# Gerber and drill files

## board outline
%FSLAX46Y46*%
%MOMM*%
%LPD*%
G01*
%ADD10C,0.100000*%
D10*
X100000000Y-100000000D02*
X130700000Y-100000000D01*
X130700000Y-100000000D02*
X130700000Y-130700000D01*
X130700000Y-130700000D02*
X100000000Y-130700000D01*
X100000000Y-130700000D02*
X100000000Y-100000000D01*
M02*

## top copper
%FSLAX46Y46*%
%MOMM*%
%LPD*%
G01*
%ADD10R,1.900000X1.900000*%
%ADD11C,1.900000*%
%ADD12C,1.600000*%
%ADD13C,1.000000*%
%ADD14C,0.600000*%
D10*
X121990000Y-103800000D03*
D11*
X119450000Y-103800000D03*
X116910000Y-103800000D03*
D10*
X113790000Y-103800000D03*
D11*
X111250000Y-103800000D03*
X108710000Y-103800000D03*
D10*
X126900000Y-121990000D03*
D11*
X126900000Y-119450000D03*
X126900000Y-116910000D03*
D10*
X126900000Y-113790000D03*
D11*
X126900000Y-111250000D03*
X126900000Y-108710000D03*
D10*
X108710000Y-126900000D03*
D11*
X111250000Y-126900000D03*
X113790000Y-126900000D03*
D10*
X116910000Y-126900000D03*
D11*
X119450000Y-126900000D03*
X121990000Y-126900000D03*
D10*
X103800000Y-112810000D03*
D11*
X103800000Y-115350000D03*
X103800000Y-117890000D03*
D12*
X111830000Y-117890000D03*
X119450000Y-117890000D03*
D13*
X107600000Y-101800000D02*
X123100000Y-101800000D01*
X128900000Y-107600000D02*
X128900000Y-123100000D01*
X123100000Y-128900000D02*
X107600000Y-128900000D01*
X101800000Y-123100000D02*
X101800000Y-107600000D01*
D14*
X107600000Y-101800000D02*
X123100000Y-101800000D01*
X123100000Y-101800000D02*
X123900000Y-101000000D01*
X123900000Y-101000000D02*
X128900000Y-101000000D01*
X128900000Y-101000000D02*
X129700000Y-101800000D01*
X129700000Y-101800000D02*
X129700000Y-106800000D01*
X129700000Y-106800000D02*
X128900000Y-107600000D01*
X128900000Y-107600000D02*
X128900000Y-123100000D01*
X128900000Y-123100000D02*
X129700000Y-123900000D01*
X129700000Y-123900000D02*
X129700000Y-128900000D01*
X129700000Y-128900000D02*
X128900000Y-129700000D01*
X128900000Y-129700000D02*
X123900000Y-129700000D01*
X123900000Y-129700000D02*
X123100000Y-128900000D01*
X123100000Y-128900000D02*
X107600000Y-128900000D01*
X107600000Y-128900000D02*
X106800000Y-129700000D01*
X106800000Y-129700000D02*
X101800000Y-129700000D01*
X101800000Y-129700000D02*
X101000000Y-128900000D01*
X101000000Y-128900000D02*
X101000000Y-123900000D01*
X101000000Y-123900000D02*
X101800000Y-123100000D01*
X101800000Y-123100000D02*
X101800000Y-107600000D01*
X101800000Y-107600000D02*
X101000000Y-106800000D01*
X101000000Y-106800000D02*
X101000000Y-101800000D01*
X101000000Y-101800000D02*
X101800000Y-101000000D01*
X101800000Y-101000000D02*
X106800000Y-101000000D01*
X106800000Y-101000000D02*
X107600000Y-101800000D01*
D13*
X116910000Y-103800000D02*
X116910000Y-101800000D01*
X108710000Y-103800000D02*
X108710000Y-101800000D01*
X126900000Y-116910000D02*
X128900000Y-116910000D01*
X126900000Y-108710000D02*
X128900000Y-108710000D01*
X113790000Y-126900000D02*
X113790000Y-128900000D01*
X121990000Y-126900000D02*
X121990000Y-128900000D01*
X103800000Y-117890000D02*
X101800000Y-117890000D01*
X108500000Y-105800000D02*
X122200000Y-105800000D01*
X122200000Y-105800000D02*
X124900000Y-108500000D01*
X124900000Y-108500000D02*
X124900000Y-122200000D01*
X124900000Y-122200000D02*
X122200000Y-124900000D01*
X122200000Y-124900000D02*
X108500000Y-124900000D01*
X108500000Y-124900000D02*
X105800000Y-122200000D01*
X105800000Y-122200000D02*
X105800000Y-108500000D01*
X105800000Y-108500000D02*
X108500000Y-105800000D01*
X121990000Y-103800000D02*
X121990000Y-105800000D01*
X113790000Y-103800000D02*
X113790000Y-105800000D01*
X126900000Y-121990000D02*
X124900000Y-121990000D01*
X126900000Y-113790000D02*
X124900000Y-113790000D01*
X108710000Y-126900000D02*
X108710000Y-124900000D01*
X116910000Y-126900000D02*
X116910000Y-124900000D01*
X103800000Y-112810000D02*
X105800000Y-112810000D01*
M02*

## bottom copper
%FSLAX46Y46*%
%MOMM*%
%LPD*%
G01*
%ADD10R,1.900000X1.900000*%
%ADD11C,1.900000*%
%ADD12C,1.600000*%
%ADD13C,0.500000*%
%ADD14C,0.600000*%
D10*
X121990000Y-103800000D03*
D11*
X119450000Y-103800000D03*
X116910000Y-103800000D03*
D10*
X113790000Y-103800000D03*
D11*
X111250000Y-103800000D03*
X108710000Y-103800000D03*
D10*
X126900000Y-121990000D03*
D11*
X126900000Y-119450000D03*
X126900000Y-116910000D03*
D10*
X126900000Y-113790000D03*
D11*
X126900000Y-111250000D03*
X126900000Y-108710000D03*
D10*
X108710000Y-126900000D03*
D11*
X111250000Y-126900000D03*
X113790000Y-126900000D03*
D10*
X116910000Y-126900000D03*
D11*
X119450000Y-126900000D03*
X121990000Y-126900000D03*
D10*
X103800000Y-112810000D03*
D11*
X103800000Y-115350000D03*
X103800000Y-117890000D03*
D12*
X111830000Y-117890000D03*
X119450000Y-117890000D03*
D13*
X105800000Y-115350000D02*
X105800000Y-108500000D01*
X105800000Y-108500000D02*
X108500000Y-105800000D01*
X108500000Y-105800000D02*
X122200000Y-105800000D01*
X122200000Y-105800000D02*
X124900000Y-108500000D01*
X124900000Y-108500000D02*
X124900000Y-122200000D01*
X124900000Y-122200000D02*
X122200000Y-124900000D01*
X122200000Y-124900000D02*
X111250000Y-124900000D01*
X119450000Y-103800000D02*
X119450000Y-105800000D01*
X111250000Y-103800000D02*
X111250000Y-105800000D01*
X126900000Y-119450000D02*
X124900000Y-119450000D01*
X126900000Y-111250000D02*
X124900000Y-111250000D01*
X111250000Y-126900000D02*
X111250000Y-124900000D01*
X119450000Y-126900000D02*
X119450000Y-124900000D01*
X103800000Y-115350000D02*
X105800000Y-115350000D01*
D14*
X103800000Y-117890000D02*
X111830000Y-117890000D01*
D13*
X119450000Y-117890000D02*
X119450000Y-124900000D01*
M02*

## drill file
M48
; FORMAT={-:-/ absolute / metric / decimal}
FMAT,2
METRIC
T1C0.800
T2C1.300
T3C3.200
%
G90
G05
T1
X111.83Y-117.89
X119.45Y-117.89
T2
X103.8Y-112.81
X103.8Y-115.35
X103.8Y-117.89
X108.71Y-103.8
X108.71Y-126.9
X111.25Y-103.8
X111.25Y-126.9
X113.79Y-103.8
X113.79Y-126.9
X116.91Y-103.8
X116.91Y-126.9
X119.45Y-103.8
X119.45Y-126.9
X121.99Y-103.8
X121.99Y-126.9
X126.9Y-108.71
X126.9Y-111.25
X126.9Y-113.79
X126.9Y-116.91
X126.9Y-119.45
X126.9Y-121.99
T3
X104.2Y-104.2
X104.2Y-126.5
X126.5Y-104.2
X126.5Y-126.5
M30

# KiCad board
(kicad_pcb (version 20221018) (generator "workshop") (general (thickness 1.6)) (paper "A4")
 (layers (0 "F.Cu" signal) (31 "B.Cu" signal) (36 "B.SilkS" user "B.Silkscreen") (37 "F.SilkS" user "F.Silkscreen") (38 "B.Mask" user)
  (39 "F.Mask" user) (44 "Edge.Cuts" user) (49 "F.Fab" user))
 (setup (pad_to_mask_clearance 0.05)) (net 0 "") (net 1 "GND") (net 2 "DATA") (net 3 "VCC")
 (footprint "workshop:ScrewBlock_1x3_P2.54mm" (layer "F.Cu") (at 121.990 103.800 180)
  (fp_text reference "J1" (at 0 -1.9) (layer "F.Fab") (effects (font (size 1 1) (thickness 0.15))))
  (pad "1" thru_hole rect (at 0.000 0 180) (size 1.9 1.9) (drill 1.3) (layers "*.Cu" "*.Mask") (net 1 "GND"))
  (pad "2" thru_hole circle (at 2.540 0 180) (size 1.9 1.9) (drill 1.3) (layers "*.Cu" "*.Mask") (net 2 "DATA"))
  (pad "3" thru_hole circle (at 5.080 0 180) (size 1.9 1.9) (drill 1.3) (layers "*.Cu" "*.Mask") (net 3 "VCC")))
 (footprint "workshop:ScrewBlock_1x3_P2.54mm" (layer "F.Cu") (at 113.790 103.800 180)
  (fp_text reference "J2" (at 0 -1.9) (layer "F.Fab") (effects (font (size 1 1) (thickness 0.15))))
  (pad "1" thru_hole rect (at 0.000 0 180) (size 1.9 1.9) (drill 1.3) (layers "*.Cu" "*.Mask") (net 1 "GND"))
  (pad "2" thru_hole circle (at 2.540 0 180) (size 1.9 1.9) (drill 1.3) (layers "*.Cu" "*.Mask") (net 2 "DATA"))
  (pad "3" thru_hole circle (at 5.080 0 180) (size 1.9 1.9) (drill 1.3) (layers "*.Cu" "*.Mask") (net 3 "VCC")))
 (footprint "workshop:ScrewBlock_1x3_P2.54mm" (layer "F.Cu") (at 126.900 121.990 90)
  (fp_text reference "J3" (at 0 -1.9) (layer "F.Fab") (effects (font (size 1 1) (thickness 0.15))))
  (pad "1" thru_hole rect (at 0.000 0 90) (size 1.9 1.9) (drill 1.3) (layers "*.Cu" "*.Mask") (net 1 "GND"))
  (pad "2" thru_hole circle (at 2.540 0 90) (size 1.9 1.9) (drill 1.3) (layers "*.Cu" "*.Mask") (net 2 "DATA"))
  (pad "3" thru_hole circle (at 5.080 0 90) (size 1.9 1.9) (drill 1.3) (layers "*.Cu" "*.Mask") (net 3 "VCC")))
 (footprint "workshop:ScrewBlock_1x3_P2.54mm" (layer "F.Cu") (at 126.900 113.790 90)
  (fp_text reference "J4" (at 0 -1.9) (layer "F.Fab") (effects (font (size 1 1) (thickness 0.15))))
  (pad "1" thru_hole rect (at 0.000 0 90) (size 1.9 1.9) (drill 1.3) (layers "*.Cu" "*.Mask") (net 1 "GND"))
  (pad "2" thru_hole circle (at 2.540 0 90) (size 1.9 1.9) (drill 1.3) (layers "*.Cu" "*.Mask") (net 2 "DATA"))
  (pad "3" thru_hole circle (at 5.080 0 90) (size 1.9 1.9) (drill 1.3) (layers "*.Cu" "*.Mask") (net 3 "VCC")))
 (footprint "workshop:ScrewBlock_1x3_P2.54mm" (layer "F.Cu") (at 108.710 126.900 0)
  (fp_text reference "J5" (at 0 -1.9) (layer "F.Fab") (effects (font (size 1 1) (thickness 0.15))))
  (pad "1" thru_hole rect (at 0.000 0 0) (size 1.9 1.9) (drill 1.3) (layers "*.Cu" "*.Mask") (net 1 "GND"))
  (pad "2" thru_hole circle (at 2.540 0 0) (size 1.9 1.9) (drill 1.3) (layers "*.Cu" "*.Mask") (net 2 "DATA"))
  (pad "3" thru_hole circle (at 5.080 0 0) (size 1.9 1.9) (drill 1.3) (layers "*.Cu" "*.Mask") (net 3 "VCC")))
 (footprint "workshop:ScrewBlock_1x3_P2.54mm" (layer "F.Cu") (at 116.910 126.900 0)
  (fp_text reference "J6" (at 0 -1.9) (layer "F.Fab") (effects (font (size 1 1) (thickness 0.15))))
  (pad "1" thru_hole rect (at 0.000 0 0) (size 1.9 1.9) (drill 1.3) (layers "*.Cu" "*.Mask") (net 1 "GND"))
  (pad "2" thru_hole circle (at 2.540 0 0) (size 1.9 1.9) (drill 1.3) (layers "*.Cu" "*.Mask") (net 2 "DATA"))
  (pad "3" thru_hole circle (at 5.080 0 0) (size 1.9 1.9) (drill 1.3) (layers "*.Cu" "*.Mask") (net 3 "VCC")))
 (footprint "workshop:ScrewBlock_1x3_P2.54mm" (layer "F.Cu") (at 103.800 112.810 270)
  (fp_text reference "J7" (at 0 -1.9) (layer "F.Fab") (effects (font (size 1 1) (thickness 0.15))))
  (pad "1" thru_hole rect (at 0.000 0 270) (size 1.9 1.9) (drill 1.3) (layers "*.Cu" "*.Mask") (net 1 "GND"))
  (pad "2" thru_hole circle (at 2.540 0 270) (size 1.9 1.9) (drill 1.3) (layers "*.Cu" "*.Mask") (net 2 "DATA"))
  (pad "3" thru_hole circle (at 5.080 0 270) (size 1.9 1.9) (drill 1.3) (layers "*.Cu" "*.Mask") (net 3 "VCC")))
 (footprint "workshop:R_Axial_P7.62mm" (layer "F.Cu") (at 111.830 117.890)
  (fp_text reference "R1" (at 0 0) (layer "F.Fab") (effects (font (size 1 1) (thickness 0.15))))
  (pad "1" thru_hole circle (at 0.000 0.000) (size 1.6 1.6) (drill 0.8) (layers "*.Cu" "*.Mask") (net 3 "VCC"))
  (pad "2" thru_hole circle (at 7.620 0.000) (size 1.6 1.6) (drill 0.8) (layers "*.Cu" "*.Mask") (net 2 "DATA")))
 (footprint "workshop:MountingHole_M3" (layer "F.Cu") (at 104.200 104.200)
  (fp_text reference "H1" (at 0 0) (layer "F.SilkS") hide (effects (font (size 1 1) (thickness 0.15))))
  (pad "" np_thru_hole circle (at 0 0) (size 3.2 3.2) (drill 3.2) (layers "*.Cu" "*.Mask")))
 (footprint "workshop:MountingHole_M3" (layer "F.Cu") (at 126.500 104.200)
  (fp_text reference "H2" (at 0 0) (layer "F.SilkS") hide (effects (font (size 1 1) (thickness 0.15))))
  (pad "" np_thru_hole circle (at 0 0) (size 3.2 3.2) (drill 3.2) (layers "*.Cu" "*.Mask")))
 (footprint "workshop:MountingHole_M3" (layer "F.Cu") (at 104.200 126.500)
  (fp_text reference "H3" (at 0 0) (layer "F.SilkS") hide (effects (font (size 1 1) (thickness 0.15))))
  (pad "" np_thru_hole circle (at 0 0) (size 3.2 3.2) (drill 3.2) (layers "*.Cu" "*.Mask")))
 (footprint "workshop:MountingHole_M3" (layer "F.Cu") (at 126.500 126.500)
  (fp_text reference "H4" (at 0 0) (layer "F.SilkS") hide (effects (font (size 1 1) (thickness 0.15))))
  (pad "" np_thru_hole circle (at 0 0) (size 3.2 3.2) (drill 3.2) (layers "*.Cu" "*.Mask")))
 (segment (start 107.600 101.800) (end 123.100 101.800) (width 1.0) (layer "F.Cu") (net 3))
 (segment (start 128.900 107.600) (end 128.900 123.100) (width 1.0) (layer "F.Cu") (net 3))
 (segment (start 123.100 128.900) (end 107.600 128.900) (width 1.0) (layer "F.Cu") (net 3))
 (segment (start 101.800 123.100) (end 101.800 107.600) (width 1.0) (layer "F.Cu") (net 3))
 (segment (start 107.600 101.800) (end 123.100 101.800) (width 0.6) (layer "F.Cu") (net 3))
 (segment (start 123.100 101.800) (end 123.900 101.000) (width 0.6) (layer "F.Cu") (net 3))
 (segment (start 123.900 101.000) (end 128.900 101.000) (width 0.6) (layer "F.Cu") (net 3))
 (segment (start 128.900 101.000) (end 129.700 101.800) (width 0.6) (layer "F.Cu") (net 3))
 (segment (start 129.700 101.800) (end 129.700 106.800) (width 0.6) (layer "F.Cu") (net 3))
 (segment (start 129.700 106.800) (end 128.900 107.600) (width 0.6) (layer "F.Cu") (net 3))
 (segment (start 128.900 107.600) (end 128.900 123.100) (width 0.6) (layer "F.Cu") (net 3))
 (segment (start 128.900 123.100) (end 129.700 123.900) (width 0.6) (layer "F.Cu") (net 3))
 (segment (start 129.700 123.900) (end 129.700 128.900) (width 0.6) (layer "F.Cu") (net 3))
 (segment (start 129.700 128.900) (end 128.900 129.700) (width 0.6) (layer "F.Cu") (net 3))
 (segment (start 128.900 129.700) (end 123.900 129.700) (width 0.6) (layer "F.Cu") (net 3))
 (segment (start 123.900 129.700) (end 123.100 128.900) (width 0.6) (layer "F.Cu") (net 3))
 (segment (start 123.100 128.900) (end 107.600 128.900) (width 0.6) (layer "F.Cu") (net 3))
 (segment (start 107.600 128.900) (end 106.800 129.700) (width 0.6) (layer "F.Cu") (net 3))
 (segment (start 106.800 129.700) (end 101.800 129.700) (width 0.6) (layer "F.Cu") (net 3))
 (segment (start 101.800 129.700) (end 101.000 128.900) (width 0.6) (layer "F.Cu") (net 3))
 (segment (start 101.000 128.900) (end 101.000 123.900) (width 0.6) (layer "F.Cu") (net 3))
 (segment (start 101.000 123.900) (end 101.800 123.100) (width 0.6) (layer "F.Cu") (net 3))
 (segment (start 101.800 123.100) (end 101.800 107.600) (width 0.6) (layer "F.Cu") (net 3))
 (segment (start 101.800 107.600) (end 101.000 106.800) (width 0.6) (layer "F.Cu") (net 3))
 (segment (start 101.000 106.800) (end 101.000 101.800) (width 0.6) (layer "F.Cu") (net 3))
 (segment (start 101.000 101.800) (end 101.800 101.000) (width 0.6) (layer "F.Cu") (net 3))
 (segment (start 101.800 101.000) (end 106.800 101.000) (width 0.6) (layer "F.Cu") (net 3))
 (segment (start 106.800 101.000) (end 107.600 101.800) (width 0.6) (layer "F.Cu") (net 3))
 (segment (start 116.910 103.800) (end 116.910 101.800) (width 1.0) (layer "F.Cu") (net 3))
 (segment (start 108.710 103.800) (end 108.710 101.800) (width 1.0) (layer "F.Cu") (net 3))
 (segment (start 126.900 116.910) (end 128.900 116.910) (width 1.0) (layer "F.Cu") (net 3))
 (segment (start 126.900 108.710) (end 128.900 108.710) (width 1.0) (layer "F.Cu") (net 3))
 (segment (start 113.790 126.900) (end 113.790 128.900) (width 1.0) (layer "F.Cu") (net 3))
 (segment (start 121.990 126.900) (end 121.990 128.900) (width 1.0) (layer "F.Cu") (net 3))
 (segment (start 103.800 117.890) (end 101.800 117.890) (width 1.0) (layer "F.Cu") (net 3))
 (segment (start 108.500 105.800) (end 122.200 105.800) (width 1.0) (layer "F.Cu") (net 1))
 (segment (start 122.200 105.800) (end 124.900 108.500) (width 1.0) (layer "F.Cu") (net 1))
 (segment (start 124.900 108.500) (end 124.900 122.200) (width 1.0) (layer "F.Cu") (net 1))
 (segment (start 124.900 122.200) (end 122.200 124.900) (width 1.0) (layer "F.Cu") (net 1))
 (segment (start 122.200 124.900) (end 108.500 124.900) (width 1.0) (layer "F.Cu") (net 1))
 (segment (start 108.500 124.900) (end 105.800 122.200) (width 1.0) (layer "F.Cu") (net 1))
 (segment (start 105.800 122.200) (end 105.800 108.500) (width 1.0) (layer "F.Cu") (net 1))
 (segment (start 105.800 108.500) (end 108.500 105.800) (width 1.0) (layer "F.Cu") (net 1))
 (segment (start 121.990 103.800) (end 121.990 105.800) (width 1.0) (layer "F.Cu") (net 1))
 (segment (start 113.790 103.800) (end 113.790 105.800) (width 1.0) (layer "F.Cu") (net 1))
 (segment (start 126.900 121.990) (end 124.900 121.990) (width 1.0) (layer "F.Cu") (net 1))
 (segment (start 126.900 113.790) (end 124.900 113.790) (width 1.0) (layer "F.Cu") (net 1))
 (segment (start 108.710 126.900) (end 108.710 124.900) (width 1.0) (layer "F.Cu") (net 1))
 (segment (start 116.910 126.900) (end 116.910 124.900) (width 1.0) (layer "F.Cu") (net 1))
 (segment (start 103.800 112.810) (end 105.800 112.810) (width 1.0) (layer "F.Cu") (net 1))
 (segment (start 105.800 115.350) (end 105.800 108.500) (width 0.5) (layer "B.Cu") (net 2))
 (segment (start 105.800 108.500) (end 108.500 105.800) (width 0.5) (layer "B.Cu") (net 2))
 (segment (start 108.500 105.800) (end 122.200 105.800) (width 0.5) (layer "B.Cu") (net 2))
 (segment (start 122.200 105.800) (end 124.900 108.500) (width 0.5) (layer "B.Cu") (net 2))
 (segment (start 124.900 108.500) (end 124.900 122.200) (width 0.5) (layer "B.Cu") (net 2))
 (segment (start 124.900 122.200) (end 122.200 124.900) (width 0.5) (layer "B.Cu") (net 2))
 (segment (start 122.200 124.900) (end 111.250 124.900) (width 0.5) (layer "B.Cu") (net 2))
 (segment (start 119.450 103.800) (end 119.450 105.800) (width 0.5) (layer "B.Cu") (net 2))
 (segment (start 111.250 103.800) (end 111.250 105.800) (width 0.5) (layer "B.Cu") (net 2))
 (segment (start 126.900 119.450) (end 124.900 119.450) (width 0.5) (layer "B.Cu") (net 2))
 (segment (start 126.900 111.250) (end 124.900 111.250) (width 0.5) (layer "B.Cu") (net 2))
 (segment (start 111.250 126.900) (end 111.250 124.900) (width 0.5) (layer "B.Cu") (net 2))
 (segment (start 119.450 126.900) (end 119.450 124.900) (width 0.5) (layer "B.Cu") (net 2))
 (segment (start 103.800 115.350) (end 105.800 115.350) (width 0.5) (layer "B.Cu") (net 2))
 (segment (start 103.800 117.890) (end 111.830 117.890) (width 0.6) (layer "B.Cu") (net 3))
 (segment (start 119.450 117.890) (end 119.450 124.900) (width 0.5) (layer "B.Cu") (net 2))
 (gr_line (start 100.000 100.000) (end 130.700 100.000) (layer "Edge.Cuts") (width 0.1))
 (gr_line (start 130.700 100.000) (end 130.700 130.700) (layer "Edge.Cuts") (width 0.1))
 (gr_line (start 130.700 130.700) (end 100.000 130.700) (layer "Edge.Cuts") (width 0.1))
 (gr_line (start 100.000 130.700) (end 100.000 100.000) (layer "Edge.Cuts") (width 0.1)))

